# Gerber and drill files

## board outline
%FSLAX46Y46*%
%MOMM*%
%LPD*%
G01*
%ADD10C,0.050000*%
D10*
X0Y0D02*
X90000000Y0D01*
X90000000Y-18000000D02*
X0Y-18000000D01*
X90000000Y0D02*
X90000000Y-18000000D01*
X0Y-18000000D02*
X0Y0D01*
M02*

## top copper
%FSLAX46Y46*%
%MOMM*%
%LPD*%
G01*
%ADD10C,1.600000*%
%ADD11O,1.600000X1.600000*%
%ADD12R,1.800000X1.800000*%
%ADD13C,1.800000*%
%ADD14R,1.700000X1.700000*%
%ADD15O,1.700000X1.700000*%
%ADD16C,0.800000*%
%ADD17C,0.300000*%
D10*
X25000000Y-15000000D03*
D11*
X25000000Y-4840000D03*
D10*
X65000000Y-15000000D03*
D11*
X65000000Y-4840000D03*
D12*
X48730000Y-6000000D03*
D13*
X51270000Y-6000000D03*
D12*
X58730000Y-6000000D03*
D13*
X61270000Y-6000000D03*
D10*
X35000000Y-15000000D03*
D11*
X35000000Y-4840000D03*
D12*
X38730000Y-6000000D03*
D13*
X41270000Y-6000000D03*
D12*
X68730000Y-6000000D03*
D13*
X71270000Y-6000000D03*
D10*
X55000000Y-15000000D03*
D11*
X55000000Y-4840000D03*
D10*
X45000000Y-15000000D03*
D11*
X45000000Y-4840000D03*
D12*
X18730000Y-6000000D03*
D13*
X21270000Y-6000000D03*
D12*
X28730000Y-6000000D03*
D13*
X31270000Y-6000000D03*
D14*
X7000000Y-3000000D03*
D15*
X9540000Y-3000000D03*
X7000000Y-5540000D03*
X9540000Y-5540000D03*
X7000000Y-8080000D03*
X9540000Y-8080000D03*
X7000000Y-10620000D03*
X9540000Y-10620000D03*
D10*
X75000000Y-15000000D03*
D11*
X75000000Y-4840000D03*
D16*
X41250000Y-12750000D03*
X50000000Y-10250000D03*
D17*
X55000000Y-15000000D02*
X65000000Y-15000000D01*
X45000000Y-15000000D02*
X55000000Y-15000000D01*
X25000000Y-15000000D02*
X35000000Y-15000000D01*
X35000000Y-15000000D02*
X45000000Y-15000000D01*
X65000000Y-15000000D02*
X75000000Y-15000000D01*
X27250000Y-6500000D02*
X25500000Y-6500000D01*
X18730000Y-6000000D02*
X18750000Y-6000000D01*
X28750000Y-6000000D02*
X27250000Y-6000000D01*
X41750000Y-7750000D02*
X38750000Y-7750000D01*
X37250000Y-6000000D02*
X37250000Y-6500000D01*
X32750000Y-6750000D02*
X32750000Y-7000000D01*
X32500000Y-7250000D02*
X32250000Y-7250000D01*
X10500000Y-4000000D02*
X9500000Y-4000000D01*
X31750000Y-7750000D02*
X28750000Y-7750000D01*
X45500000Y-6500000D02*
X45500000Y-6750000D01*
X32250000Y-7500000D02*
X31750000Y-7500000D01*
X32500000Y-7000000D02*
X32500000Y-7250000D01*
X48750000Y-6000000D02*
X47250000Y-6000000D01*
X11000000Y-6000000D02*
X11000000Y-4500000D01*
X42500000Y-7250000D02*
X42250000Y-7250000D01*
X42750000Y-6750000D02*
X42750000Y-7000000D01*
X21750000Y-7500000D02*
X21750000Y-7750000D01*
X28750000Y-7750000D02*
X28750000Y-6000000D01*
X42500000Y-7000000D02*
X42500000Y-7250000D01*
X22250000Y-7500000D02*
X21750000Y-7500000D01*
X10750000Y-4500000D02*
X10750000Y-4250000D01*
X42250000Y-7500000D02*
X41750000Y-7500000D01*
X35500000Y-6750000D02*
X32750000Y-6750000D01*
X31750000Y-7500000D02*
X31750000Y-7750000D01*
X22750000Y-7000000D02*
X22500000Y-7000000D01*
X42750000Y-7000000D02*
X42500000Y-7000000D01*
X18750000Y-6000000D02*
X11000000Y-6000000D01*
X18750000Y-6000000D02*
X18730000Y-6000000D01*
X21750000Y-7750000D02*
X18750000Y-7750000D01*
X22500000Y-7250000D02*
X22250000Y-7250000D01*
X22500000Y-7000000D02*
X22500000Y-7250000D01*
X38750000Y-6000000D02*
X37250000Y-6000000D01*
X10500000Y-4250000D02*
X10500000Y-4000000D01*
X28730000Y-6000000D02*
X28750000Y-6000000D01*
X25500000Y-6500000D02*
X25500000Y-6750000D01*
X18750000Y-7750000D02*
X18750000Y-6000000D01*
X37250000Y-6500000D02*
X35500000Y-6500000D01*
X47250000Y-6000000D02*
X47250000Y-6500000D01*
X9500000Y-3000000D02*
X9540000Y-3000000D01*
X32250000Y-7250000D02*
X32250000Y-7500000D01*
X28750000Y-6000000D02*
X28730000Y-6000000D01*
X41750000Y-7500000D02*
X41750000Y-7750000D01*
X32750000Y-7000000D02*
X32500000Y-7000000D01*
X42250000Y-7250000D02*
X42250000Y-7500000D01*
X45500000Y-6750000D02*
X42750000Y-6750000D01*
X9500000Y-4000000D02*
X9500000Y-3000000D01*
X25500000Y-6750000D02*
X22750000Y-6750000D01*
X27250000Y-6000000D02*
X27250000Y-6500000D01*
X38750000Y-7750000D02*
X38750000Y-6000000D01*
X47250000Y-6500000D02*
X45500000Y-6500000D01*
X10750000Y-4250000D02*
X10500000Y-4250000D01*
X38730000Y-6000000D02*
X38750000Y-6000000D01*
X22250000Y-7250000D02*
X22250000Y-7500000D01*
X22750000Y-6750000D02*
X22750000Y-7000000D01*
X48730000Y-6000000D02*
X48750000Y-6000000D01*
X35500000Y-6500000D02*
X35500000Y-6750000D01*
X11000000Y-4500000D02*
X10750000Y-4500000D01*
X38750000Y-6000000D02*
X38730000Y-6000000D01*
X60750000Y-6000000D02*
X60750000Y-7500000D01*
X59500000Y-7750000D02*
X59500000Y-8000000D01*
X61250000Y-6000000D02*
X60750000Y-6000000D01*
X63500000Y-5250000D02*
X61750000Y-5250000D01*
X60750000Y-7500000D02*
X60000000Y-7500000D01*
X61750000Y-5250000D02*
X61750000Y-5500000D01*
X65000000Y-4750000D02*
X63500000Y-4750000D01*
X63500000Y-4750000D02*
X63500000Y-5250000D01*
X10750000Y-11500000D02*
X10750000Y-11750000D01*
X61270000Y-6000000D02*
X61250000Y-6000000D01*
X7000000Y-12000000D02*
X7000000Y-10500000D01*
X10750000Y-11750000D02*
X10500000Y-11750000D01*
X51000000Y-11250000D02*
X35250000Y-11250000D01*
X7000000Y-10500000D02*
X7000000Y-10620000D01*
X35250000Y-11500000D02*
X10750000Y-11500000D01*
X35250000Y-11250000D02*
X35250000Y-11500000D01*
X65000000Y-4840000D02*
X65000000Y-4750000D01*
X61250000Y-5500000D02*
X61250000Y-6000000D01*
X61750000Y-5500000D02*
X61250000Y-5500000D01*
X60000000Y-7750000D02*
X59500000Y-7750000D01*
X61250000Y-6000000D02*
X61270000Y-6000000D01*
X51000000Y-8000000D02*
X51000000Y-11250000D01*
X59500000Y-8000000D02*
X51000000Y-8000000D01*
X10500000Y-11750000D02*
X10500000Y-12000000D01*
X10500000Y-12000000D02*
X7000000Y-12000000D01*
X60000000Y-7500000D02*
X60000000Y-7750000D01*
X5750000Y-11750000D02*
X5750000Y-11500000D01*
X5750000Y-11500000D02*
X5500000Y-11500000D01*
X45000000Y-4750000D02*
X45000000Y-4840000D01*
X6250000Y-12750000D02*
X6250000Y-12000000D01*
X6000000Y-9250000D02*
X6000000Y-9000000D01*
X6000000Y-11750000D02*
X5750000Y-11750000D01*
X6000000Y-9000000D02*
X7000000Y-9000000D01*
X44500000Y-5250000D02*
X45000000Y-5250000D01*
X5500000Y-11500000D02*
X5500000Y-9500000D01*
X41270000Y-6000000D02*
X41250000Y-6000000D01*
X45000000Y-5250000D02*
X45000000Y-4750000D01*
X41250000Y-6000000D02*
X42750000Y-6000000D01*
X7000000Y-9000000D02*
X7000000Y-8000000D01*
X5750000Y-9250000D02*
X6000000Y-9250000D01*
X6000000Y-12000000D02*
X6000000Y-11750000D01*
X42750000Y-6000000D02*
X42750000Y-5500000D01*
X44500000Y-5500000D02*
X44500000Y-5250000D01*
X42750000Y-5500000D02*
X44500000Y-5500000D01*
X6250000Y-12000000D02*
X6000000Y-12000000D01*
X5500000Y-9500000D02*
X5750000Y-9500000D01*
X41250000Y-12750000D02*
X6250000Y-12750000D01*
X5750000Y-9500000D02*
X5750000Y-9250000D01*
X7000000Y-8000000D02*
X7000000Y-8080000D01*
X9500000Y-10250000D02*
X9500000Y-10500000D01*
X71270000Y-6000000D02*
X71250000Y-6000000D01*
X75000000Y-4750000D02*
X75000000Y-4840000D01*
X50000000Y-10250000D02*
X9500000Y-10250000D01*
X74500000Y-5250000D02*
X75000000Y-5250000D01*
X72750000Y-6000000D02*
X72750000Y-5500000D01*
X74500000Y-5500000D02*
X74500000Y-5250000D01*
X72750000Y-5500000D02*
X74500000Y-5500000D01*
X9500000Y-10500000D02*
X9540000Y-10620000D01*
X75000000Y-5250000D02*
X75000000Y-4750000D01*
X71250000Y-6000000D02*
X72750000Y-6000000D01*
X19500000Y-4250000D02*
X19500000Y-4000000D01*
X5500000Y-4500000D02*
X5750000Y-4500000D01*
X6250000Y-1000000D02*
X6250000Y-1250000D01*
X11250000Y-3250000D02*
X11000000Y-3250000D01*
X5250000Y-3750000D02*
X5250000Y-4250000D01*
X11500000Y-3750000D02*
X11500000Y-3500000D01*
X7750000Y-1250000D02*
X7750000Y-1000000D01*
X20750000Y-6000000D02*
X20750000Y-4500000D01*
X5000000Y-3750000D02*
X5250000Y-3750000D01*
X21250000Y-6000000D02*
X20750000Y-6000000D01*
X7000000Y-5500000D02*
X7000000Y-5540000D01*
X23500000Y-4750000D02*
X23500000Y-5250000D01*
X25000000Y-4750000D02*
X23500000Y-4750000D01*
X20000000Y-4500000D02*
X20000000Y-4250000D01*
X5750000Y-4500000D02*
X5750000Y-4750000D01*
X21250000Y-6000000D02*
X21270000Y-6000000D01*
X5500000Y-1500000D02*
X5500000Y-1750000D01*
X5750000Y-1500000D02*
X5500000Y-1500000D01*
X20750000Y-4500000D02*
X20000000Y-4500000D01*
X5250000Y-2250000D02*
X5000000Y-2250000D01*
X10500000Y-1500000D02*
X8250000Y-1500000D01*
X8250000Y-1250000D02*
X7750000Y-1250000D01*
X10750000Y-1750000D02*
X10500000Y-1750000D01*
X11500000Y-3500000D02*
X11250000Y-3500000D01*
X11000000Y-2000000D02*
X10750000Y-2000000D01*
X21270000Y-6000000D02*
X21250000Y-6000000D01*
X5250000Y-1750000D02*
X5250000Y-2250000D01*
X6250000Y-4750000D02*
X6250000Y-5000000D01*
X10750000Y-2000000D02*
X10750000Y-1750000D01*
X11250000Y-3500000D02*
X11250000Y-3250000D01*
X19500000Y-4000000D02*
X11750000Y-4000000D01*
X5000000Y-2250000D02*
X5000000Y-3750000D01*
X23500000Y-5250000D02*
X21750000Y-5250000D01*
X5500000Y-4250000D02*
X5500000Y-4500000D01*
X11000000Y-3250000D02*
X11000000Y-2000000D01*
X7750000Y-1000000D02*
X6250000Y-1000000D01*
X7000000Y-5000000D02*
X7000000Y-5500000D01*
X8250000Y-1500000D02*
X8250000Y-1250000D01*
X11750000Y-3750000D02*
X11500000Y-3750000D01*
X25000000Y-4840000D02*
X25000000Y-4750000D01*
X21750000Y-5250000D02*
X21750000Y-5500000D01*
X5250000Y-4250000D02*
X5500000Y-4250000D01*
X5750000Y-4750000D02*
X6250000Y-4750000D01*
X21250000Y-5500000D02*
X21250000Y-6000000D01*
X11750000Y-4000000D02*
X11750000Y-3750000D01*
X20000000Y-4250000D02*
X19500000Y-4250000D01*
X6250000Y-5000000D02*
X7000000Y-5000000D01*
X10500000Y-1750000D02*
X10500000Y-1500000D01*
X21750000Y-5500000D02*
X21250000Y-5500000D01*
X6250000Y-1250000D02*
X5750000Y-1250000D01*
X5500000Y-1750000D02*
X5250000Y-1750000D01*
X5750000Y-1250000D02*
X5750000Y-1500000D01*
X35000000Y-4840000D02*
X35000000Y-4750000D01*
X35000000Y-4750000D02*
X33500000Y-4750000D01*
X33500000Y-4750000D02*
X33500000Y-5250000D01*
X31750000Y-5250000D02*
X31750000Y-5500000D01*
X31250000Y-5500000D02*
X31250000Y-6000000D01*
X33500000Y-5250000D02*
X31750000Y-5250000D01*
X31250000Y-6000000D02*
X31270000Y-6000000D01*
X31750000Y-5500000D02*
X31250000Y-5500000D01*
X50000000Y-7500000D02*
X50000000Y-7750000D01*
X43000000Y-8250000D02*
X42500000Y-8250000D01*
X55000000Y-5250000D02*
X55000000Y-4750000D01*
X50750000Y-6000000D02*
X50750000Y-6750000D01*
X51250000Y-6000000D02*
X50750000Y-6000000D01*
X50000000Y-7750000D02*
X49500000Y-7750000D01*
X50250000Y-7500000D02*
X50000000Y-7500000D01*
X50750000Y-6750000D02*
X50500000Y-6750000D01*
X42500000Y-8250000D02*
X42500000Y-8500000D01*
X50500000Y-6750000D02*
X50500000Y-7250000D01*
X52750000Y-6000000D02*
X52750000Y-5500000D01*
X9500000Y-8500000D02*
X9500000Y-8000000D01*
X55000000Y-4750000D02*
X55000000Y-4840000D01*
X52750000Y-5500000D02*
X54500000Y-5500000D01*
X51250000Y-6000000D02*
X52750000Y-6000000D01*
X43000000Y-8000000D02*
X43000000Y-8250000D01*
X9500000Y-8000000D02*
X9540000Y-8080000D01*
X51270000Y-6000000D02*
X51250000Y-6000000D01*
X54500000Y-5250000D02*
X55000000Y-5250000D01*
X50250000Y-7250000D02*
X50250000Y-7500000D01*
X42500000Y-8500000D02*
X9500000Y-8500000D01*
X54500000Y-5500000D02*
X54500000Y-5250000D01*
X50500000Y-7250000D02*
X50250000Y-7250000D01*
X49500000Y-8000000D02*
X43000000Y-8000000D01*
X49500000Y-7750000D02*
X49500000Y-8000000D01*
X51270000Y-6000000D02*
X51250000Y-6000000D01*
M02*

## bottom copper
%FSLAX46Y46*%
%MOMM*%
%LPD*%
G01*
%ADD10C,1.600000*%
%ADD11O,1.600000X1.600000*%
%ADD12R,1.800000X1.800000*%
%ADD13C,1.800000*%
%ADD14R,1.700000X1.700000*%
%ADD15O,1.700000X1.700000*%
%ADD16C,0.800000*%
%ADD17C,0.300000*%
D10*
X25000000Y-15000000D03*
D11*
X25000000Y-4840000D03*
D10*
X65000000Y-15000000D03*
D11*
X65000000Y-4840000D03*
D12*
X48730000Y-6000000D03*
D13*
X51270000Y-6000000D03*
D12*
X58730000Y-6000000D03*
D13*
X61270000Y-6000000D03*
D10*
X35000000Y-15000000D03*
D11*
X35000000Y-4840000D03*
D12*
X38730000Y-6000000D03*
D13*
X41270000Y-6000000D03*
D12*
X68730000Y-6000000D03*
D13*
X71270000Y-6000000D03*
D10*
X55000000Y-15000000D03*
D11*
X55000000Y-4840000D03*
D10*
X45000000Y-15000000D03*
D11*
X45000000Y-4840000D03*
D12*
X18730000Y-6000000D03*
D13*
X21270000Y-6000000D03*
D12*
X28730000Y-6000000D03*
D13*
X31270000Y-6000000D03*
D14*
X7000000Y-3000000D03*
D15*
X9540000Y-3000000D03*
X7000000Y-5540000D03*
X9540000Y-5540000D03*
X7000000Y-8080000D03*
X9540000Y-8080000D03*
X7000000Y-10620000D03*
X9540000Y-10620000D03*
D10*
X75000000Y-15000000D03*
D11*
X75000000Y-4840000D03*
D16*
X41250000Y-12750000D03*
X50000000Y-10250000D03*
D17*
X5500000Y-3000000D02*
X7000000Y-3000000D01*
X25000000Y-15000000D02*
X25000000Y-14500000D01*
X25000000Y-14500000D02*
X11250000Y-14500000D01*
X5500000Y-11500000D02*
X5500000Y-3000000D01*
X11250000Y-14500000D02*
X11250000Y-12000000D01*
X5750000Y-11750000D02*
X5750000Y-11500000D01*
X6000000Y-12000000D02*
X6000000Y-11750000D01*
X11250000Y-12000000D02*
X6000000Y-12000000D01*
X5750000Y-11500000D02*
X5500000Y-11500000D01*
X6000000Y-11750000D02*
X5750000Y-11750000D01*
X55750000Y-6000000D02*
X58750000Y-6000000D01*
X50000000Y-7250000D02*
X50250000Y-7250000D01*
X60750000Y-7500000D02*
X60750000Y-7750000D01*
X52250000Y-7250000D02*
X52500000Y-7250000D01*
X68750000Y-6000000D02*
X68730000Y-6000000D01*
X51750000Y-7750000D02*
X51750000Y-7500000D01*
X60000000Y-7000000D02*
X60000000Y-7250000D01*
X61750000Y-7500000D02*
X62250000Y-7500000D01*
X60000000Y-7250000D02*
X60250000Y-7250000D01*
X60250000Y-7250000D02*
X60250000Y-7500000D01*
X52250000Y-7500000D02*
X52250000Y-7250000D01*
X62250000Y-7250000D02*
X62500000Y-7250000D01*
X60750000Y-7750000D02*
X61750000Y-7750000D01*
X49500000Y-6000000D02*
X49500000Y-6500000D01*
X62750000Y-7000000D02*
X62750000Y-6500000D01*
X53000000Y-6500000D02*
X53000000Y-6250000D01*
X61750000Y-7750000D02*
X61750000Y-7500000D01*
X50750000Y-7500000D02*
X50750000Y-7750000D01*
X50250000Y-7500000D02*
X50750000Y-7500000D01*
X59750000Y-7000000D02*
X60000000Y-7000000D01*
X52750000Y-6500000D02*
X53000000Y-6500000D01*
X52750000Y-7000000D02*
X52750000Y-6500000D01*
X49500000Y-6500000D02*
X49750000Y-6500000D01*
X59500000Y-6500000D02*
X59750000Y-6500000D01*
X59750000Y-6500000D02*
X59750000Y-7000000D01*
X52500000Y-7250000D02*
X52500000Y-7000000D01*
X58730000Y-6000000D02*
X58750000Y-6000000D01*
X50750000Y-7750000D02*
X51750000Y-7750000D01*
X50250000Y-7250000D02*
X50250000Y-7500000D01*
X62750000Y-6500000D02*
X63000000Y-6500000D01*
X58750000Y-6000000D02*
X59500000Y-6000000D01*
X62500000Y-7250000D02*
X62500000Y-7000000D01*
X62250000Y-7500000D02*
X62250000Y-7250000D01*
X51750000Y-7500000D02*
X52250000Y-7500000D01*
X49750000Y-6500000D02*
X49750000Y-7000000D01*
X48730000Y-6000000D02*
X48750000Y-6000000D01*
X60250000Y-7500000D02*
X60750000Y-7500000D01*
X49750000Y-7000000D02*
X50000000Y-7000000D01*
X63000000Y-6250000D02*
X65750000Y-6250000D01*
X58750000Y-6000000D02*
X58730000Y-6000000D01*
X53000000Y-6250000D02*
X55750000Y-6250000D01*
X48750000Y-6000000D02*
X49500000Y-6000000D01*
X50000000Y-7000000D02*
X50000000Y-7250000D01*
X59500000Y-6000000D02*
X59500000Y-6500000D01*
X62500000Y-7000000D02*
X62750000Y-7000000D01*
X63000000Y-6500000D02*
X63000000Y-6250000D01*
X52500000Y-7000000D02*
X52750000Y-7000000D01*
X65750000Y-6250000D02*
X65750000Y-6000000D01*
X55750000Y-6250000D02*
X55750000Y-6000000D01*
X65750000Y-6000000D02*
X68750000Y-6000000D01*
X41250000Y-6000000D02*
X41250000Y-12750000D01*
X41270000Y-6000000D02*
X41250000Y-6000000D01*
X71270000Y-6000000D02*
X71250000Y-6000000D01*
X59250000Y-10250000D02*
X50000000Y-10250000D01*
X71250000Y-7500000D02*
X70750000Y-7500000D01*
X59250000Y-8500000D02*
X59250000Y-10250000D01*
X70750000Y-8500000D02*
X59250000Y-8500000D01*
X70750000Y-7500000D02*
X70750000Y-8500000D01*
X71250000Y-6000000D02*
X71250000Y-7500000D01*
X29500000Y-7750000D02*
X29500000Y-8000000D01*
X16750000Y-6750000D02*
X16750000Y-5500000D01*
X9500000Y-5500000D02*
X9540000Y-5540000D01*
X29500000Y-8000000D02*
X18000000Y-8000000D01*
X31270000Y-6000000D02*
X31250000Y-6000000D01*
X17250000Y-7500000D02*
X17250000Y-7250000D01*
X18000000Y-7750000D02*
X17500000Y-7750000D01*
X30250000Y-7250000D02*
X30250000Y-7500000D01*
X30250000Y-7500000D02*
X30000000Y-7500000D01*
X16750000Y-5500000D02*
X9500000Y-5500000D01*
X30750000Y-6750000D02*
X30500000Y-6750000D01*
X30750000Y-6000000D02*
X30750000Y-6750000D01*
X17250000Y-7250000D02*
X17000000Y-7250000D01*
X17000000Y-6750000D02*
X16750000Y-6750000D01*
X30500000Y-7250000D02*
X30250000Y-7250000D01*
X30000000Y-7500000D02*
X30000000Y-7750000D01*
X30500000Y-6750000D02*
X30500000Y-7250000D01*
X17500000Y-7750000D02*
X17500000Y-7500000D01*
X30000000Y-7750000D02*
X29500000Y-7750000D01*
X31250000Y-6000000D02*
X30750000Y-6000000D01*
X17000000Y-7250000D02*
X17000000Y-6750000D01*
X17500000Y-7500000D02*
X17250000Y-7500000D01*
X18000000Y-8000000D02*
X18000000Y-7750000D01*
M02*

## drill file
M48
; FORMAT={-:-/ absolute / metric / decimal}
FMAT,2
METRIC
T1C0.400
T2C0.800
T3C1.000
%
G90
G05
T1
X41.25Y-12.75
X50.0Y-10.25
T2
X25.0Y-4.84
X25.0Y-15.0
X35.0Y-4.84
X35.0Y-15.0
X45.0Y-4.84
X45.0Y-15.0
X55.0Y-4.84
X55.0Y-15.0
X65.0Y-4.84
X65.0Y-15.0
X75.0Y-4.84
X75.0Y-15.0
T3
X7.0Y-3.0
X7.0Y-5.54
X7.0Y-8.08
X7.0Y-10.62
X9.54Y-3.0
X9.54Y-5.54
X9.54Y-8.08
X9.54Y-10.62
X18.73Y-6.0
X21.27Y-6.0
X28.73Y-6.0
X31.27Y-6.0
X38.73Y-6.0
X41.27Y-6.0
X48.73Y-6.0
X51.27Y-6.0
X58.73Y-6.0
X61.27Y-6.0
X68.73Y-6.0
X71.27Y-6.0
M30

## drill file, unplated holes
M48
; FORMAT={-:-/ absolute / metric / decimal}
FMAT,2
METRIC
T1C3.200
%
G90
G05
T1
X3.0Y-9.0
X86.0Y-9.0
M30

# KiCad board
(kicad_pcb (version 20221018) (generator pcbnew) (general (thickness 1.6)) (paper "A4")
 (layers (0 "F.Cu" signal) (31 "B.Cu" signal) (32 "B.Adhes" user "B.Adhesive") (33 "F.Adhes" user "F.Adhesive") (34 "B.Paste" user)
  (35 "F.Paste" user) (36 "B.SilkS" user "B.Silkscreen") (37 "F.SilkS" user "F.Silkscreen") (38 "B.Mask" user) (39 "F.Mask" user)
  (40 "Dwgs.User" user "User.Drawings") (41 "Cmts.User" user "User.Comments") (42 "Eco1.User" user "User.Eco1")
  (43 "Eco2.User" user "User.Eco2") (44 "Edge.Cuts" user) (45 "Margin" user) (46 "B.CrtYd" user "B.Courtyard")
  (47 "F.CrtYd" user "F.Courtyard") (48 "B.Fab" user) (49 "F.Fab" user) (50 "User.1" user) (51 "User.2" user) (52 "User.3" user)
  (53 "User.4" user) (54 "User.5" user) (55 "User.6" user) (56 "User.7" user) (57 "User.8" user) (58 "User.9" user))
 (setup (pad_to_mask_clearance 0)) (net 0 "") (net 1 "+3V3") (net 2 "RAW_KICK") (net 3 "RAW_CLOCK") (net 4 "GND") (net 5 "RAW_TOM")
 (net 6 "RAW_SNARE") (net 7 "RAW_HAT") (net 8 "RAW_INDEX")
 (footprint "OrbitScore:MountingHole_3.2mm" (layer "F.Cu") (at 3 9)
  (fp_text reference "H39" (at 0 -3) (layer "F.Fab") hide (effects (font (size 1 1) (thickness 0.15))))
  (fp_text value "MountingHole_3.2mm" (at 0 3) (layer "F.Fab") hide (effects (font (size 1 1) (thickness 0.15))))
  (pad "" np_thru_hole circle (at 0 0) (size 3.2 3.2) (drill 3.2) (layers "*.Cu" "*.Mask")))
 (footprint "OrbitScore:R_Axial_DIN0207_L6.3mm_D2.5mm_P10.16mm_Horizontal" (layer "F.Cu") (at 25 15 90)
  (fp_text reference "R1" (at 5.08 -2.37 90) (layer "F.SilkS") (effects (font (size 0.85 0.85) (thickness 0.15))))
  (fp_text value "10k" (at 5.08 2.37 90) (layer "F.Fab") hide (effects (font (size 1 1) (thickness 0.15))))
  (pad "1" thru_hole circle (at 0 0 90) (size 1.6 1.6) (drill 0.8) (layers "*.Cu" "*.Mask") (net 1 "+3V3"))
  (pad "2" thru_hole oval (at 10.16 0 90) (size 1.6 1.6) (drill 0.8) (layers "*.Cu" "*.Mask") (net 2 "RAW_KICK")))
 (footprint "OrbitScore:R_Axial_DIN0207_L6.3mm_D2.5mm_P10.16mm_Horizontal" (layer "F.Cu") (at 65 15 90)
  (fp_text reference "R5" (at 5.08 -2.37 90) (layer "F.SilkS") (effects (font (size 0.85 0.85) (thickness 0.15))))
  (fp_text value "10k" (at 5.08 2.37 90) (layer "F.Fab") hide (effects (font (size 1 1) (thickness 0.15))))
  (pad "1" thru_hole circle (at 0 0 90) (size 1.6 1.6) (drill 0.8) (layers "*.Cu" "*.Mask") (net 1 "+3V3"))
  (pad "2" thru_hole oval (at 10.16 0 90) (size 1.6 1.6) (drill 0.8) (layers "*.Cu" "*.Mask") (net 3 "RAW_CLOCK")))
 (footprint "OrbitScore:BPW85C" (layer "F.Cu") (at 50 6)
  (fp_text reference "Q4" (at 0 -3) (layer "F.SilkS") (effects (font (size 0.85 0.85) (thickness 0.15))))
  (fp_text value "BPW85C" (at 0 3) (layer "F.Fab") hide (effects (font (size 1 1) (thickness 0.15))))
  (pad "1" thru_hole rect (at -1.27 0) (size 1.8 1.8) (drill 1) (layers "*.Cu" "*.Mask") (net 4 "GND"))
  (pad "2" thru_hole circle (at 1.27 0) (size 1.8 1.8) (drill 1) (layers "*.Cu" "*.Mask") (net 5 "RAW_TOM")))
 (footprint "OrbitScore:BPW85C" (layer "F.Cu") (at 60 6)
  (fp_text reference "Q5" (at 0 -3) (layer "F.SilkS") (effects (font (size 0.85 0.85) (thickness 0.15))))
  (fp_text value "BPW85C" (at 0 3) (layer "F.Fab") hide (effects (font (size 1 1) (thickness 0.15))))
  (pad "1" thru_hole rect (at -1.27 0) (size 1.8 1.8) (drill 1) (layers "*.Cu" "*.Mask") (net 4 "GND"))
  (pad "2" thru_hole circle (at 1.27 0) (size 1.8 1.8) (drill 1) (layers "*.Cu" "*.Mask") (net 3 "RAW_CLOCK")))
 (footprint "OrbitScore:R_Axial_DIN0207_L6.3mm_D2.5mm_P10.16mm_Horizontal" (layer "F.Cu") (at 35 15 90)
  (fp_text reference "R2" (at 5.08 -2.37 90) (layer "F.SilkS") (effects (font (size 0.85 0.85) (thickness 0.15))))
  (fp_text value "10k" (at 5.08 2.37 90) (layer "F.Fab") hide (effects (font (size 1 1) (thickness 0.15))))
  (pad "1" thru_hole circle (at 0 0 90) (size 1.6 1.6) (drill 0.8) (layers "*.Cu" "*.Mask") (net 1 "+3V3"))
  (pad "2" thru_hole oval (at 10.16 0 90) (size 1.6 1.6) (drill 0.8) (layers "*.Cu" "*.Mask") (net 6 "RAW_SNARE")))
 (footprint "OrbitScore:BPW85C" (layer "F.Cu") (at 40 6)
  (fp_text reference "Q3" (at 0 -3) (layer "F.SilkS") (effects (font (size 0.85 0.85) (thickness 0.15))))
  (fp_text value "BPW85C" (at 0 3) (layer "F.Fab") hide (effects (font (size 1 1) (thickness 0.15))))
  (pad "1" thru_hole rect (at -1.27 0) (size 1.8 1.8) (drill 1) (layers "*.Cu" "*.Mask") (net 4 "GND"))
  (pad "2" thru_hole circle (at 1.27 0) (size 1.8 1.8) (drill 1) (layers "*.Cu" "*.Mask") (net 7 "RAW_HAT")))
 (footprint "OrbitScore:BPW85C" (layer "F.Cu") (at 70 6)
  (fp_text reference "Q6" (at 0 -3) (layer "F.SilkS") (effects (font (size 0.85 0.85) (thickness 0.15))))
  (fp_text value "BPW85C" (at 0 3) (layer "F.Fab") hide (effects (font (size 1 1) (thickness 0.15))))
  (pad "1" thru_hole rect (at -1.27 0) (size 1.8 1.8) (drill 1) (layers "*.Cu" "*.Mask") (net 4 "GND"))
  (pad "2" thru_hole circle (at 1.27 0) (size 1.8 1.8) (drill 1) (layers "*.Cu" "*.Mask") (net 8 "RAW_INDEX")))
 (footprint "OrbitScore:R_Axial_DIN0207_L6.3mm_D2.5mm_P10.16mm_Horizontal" (layer "F.Cu") (at 55 15 90)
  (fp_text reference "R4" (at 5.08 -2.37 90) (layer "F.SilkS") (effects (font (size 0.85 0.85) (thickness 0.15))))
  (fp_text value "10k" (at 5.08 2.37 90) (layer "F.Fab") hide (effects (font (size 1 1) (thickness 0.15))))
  (pad "1" thru_hole circle (at 0 0 90) (size 1.6 1.6) (drill 0.8) (layers "*.Cu" "*.Mask") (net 1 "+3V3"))
  (pad "2" thru_hole oval (at 10.16 0 90) (size 1.6 1.6) (drill 0.8) (layers "*.Cu" "*.Mask") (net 5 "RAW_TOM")))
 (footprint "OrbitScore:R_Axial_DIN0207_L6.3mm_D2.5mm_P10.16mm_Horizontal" (layer "F.Cu") (at 45 15 90)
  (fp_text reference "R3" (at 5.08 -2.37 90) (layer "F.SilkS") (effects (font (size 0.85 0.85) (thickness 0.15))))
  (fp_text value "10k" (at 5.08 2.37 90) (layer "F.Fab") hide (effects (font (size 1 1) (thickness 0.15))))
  (pad "1" thru_hole circle (at 0 0 90) (size 1.6 1.6) (drill 0.8) (layers "*.Cu" "*.Mask") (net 1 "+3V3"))
  (pad "2" thru_hole oval (at 10.16 0 90) (size 1.6 1.6) (drill 0.8) (layers "*.Cu" "*.Mask") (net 7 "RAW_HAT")))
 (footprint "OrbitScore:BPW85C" (layer "F.Cu") (at 20 6)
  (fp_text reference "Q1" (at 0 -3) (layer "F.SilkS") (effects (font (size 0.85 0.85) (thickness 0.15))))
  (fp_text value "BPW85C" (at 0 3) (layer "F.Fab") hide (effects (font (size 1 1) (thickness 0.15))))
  (pad "1" thru_hole rect (at -1.27 0) (size 1.8 1.8) (drill 1) (layers "*.Cu" "*.Mask") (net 4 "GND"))
  (pad "2" thru_hole circle (at 1.27 0) (size 1.8 1.8) (drill 1) (layers "*.Cu" "*.Mask") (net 2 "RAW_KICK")))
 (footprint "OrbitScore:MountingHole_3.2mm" (layer "F.Cu") (at 86 9)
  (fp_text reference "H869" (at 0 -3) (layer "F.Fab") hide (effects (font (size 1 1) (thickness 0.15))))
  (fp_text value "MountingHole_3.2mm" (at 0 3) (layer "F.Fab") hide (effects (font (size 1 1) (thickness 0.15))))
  (pad "" np_thru_hole circle (at 0 0) (size 3.2 3.2) (drill 3.2) (layers "*.Cu" "*.Mask")))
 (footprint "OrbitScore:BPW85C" (layer "F.Cu") (at 30 6)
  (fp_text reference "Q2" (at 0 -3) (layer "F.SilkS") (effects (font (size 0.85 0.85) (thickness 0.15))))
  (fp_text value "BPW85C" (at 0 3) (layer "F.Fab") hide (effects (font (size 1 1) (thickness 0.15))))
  (pad "1" thru_hole rect (at -1.27 0) (size 1.8 1.8) (drill 1) (layers "*.Cu" "*.Mask") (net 4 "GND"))
  (pad "2" thru_hole circle (at 1.27 0) (size 1.8 1.8) (drill 1) (layers "*.Cu" "*.Mask") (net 6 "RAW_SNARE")))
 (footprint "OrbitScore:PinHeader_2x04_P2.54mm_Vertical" (layer "F.Cu") (at 7 3)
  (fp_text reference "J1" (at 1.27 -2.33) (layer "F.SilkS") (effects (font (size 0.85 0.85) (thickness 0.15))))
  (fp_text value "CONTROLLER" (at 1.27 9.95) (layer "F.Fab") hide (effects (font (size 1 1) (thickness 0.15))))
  (pad "1" thru_hole rect (at 0 0) (size 1.7 1.7) (drill 1) (layers "*.Cu" "*.Mask") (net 1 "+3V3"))
  (pad "2" thru_hole oval (at 2.54 0) (size 1.7 1.7) (drill 1) (layers "*.Cu" "*.Mask") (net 4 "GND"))
  (pad "3" thru_hole oval (at 0 2.54) (size 1.7 1.7) (drill 1) (layers "*.Cu" "*.Mask") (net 2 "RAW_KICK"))
  (pad "4" thru_hole oval (at 2.54 2.54) (size 1.7 1.7) (drill 1) (layers "*.Cu" "*.Mask") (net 6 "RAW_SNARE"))
  (pad "5" thru_hole oval (at 0 5.08) (size 1.7 1.7) (drill 1) (layers "*.Cu" "*.Mask") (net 7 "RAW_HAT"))
  (pad "6" thru_hole oval (at 2.54 5.08) (size 1.7 1.7) (drill 1) (layers "*.Cu" "*.Mask") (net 5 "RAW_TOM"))
  (pad "7" thru_hole oval (at 0 7.62) (size 1.7 1.7) (drill 1) (layers "*.Cu" "*.Mask") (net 3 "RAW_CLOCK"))
  (pad "8" thru_hole oval (at 2.54 7.62) (size 1.7 1.7) (drill 1) (layers "*.Cu" "*.Mask") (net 8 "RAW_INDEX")))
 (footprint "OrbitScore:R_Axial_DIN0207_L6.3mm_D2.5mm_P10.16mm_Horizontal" (layer "F.Cu") (at 75 15 90)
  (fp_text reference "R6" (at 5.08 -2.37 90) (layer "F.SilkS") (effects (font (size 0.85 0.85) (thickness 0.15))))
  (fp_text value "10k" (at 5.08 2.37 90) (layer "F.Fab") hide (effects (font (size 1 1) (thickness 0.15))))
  (pad "1" thru_hole circle (at 0 0 90) (size 1.6 1.6) (drill 0.8) (layers "*.Cu" "*.Mask") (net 1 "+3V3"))
  (pad "2" thru_hole oval (at 10.16 0 90) (size 1.6 1.6) (drill 0.8) (layers "*.Cu" "*.Mask") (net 8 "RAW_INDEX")))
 (gr_line (start 0 0) (end 90 0) (stroke (width 0.05) (type default)) (layer "Edge.Cuts"))
 (gr_line (start 90 18) (end 0 18) (stroke (width 0.05) (type default)) (layer "Edge.Cuts"))
 (gr_line (start 90 0) (end 90 18) (stroke (width 0.05) (type default)) (layer "Edge.Cuts"))
 (gr_line (start 0 18) (end 0 0) (stroke (width 0.05) (type default)) (layer "Edge.Cuts"))
 (segment (start 55 15) (end 65 15) (width 0.3) (layer "F.Cu") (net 1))
 (segment (start 45 15) (end 55 15) (width 0.3) (layer "F.Cu") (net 1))
 (segment (start 25 15) (end 35 15) (width 0.3) (layer "F.Cu") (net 1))
 (segment (start 35 15) (end 45 15) (width 0.3) (layer "F.Cu") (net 1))
 (segment (start 65 15) (end 75 15) (width 0.3) (layer "F.Cu") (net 1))
 (segment (start 5.5 3) (end 7 3) (width 0.3) (layer "B.Cu") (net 1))
 (segment (start 25 15) (end 25 14.5) (width 0.3) (layer "B.Cu") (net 1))
 (segment (start 25 14.5) (end 11.25 14.5) (width 0.3) (layer "B.Cu") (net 1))
 (segment (start 5.5 11.5) (end 5.5 3) (width 0.3) (layer "B.Cu") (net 1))
 (segment (start 11.25 14.5) (end 11.25 12) (width 0.3) (layer "B.Cu") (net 1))
 (segment (start 5.75 11.75) (end 5.75 11.5) (width 0.3) (layer "B.Cu") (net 1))
 (segment (start 6 12) (end 6 11.75) (width 0.3) (layer "B.Cu") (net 1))
 (segment (start 11.25 12) (end 6 12) (width 0.3) (layer "B.Cu") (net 1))
 (segment (start 5.75 11.5) (end 5.5 11.5) (width 0.3) (layer "B.Cu") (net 1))
 (segment (start 6 11.75) (end 5.75 11.75) (width 0.3) (layer "B.Cu") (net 1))
 (segment (start 27.25 6.5) (end 25.5 6.5) (width 0.3) (layer "F.Cu") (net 4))
 (segment (start 18.73 6) (end 18.75 6) (width 0.3) (layer "F.Cu") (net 4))
 (segment (start 28.75 6) (end 27.25 6) (width 0.3) (layer "F.Cu") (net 4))
 (segment (start 41.75 7.75) (end 38.75 7.75) (width 0.3) (layer "F.Cu") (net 4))
 (segment (start 37.25 6) (end 37.25 6.5) (width 0.3) (layer "F.Cu") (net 4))
 (segment (start 32.75 6.75) (end 32.75 7) (width 0.3) (layer "F.Cu") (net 4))
 (segment (start 32.5 7.25) (end 32.25 7.25) (width 0.3) (layer "F.Cu") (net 4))
 (segment (start 10.5 4) (end 9.5 4) (width 0.3) (layer "F.Cu") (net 4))
 (segment (start 31.75 7.75) (end 28.75 7.75) (width 0.3) (layer "F.Cu") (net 4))
 (segment (start 45.5 6.5) (end 45.5 6.75) (width 0.3) (layer "F.Cu") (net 4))
 (segment (start 32.25 7.5) (end 31.75 7.5) (width 0.3) (layer "F.Cu") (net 4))
 (segment (start 32.5 7) (end 32.5 7.25) (width 0.3) (layer "F.Cu") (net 4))
 (segment (start 48.75 6) (end 47.25 6) (width 0.3) (layer "F.Cu") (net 4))
 (segment (start 11 6) (end 11 4.5) (width 0.3) (layer "F.Cu") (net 4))
 (segment (start 42.5 7.25) (end 42.25 7.25) (width 0.3) (layer "F.Cu") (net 4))
 (segment (start 42.75 6.75) (end 42.75 7) (width 0.3) (layer "F.Cu") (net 4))
 (segment (start 21.75 7.5) (end 21.75 7.75) (width 0.3) (layer "F.Cu") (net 4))
 (segment (start 28.75 7.75) (end 28.75 6) (width 0.3) (layer "F.Cu") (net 4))
 (segment (start 42.5 7) (end 42.5 7.25) (width 0.3) (layer "F.Cu") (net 4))
 (segment (start 22.25 7.5) (end 21.75 7.5) (width 0.3) (layer "F.Cu") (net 4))
 (segment (start 10.75 4.5) (end 10.75 4.25) (width 0.3) (layer "F.Cu") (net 4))
 (segment (start 42.25 7.5) (end 41.75 7.5) (width 0.3) (layer "F.Cu") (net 4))
 (segment (start 35.5 6.75) (end 32.75 6.75) (width 0.3) (layer "F.Cu") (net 4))
 (segment (start 31.75 7.5) (end 31.75 7.75) (width 0.3) (layer "F.Cu") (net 4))
 (segment (start 22.75 7) (end 22.5 7) (width 0.3) (layer "F.Cu") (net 4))
 (segment (start 42.75 7) (end 42.5 7) (width 0.3) (layer "F.Cu") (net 4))
 (segment (start 18.75 6) (end 11 6) (width 0.3) (layer "F.Cu") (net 4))
 (segment (start 18.75 6) (end 18.73 6) (width 0.3) (layer "F.Cu") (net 4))
 (segment (start 21.75 7.75) (end 18.75 7.75) (width 0.3) (layer "F.Cu") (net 4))
 (segment (start 22.5 7.25) (end 22.25 7.25) (width 0.3) (layer "F.Cu") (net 4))
 (segment (start 22.5 7) (end 22.5 7.25) (width 0.3) (layer "F.Cu") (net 4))
 (segment (start 38.75 6) (end 37.25 6) (width 0.3) (layer "F.Cu") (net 4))
 (segment (start 10.5 4.25) (end 10.5 4) (width 0.3) (layer "F.Cu") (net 4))
 (segment (start 28.73 6) (end 28.75 6) (width 0.3) (layer "F.Cu") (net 4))
 (segment (start 25.5 6.5) (end 25.5 6.75) (width 0.3) (layer "F.Cu") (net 4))
 (segment (start 18.75 7.75) (end 18.75 6) (width 0.3) (layer "F.Cu") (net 4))
 (segment (start 37.25 6.5) (end 35.5 6.5) (width 0.3) (layer "F.Cu") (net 4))
 (segment (start 47.25 6) (end 47.25 6.5) (width 0.3) (layer "F.Cu") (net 4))
 (segment (start 9.5 3) (end 9.54 3) (width 0.3) (layer "F.Cu") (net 4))
 (segment (start 32.25 7.25) (end 32.25 7.5) (width 0.3) (layer "F.Cu") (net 4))
 (segment (start 28.75 6) (end 28.73 6) (width 0.3) (layer "F.Cu") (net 4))
 (segment (start 41.75 7.5) (end 41.75 7.75) (width 0.3) (layer "F.Cu") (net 4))
 (segment (start 32.75 7) (end 32.5 7) (width 0.3) (layer "F.Cu") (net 4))
 (segment (start 42.25 7.25) (end 42.25 7.5) (width 0.3) (layer "F.Cu") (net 4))
 (segment (start 45.5 6.75) (end 42.75 6.75) (width 0.3) (layer "F.Cu") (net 4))
 (segment (start 9.5 4) (end 9.5 3) (width 0.3) (layer "F.Cu") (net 4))
 (segment (start 25.5 6.75) (end 22.75 6.75) (width 0.3) (layer "F.Cu") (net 4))
 (segment (start 27.25 6) (end 27.25 6.5) (width 0.3) (layer "F.Cu") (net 4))
 (segment (start 38.75 7.75) (end 38.75 6) (width 0.3) (layer "F.Cu") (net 4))
 (segment (start 47.25 6.5) (end 45.5 6.5) (width 0.3) (layer "F.Cu") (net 4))
 (segment (start 10.75 4.25) (end 10.5 4.25) (width 0.3) (layer "F.Cu") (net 4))
 (segment (start 38.73 6) (end 38.75 6) (width 0.3) (layer "F.Cu") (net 4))
 (segment (start 22.25 7.25) (end 22.25 7.5) (width 0.3) (layer "F.Cu") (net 4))
 (segment (start 22.75 6.75) (end 22.75 7) (width 0.3) (layer "F.Cu") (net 4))
 (segment (start 48.73 6) (end 48.75 6) (width 0.3) (layer "F.Cu") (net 4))
 (segment (start 35.5 6.5) (end 35.5 6.75) (width 0.3) (layer "F.Cu") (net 4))
 (segment (start 11 4.5) (end 10.75 4.5) (width 0.3) (layer "F.Cu") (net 4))
 (segment (start 38.75 6) (end 38.73 6) (width 0.3) (layer "F.Cu") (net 4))
 (segment (start 55.75 6) (end 58.75 6) (width 0.3) (layer "B.Cu") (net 4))
 (segment (start 50 7.25) (end 50.25 7.25) (width 0.3) (layer "B.Cu") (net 4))
 (segment (start 60.75 7.5) (end 60.75 7.75) (width 0.3) (layer "B.Cu") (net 4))
 (segment (start 52.25 7.25) (end 52.5 7.25) (width 0.3) (layer "B.Cu") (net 4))
 (segment (start 68.75 6) (end 68.73 6) (width 0.3) (layer "B.Cu") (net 4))
 (segment (start 51.75 7.75) (end 51.75 7.5) (width 0.3) (layer "B.Cu") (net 4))
 (segment (start 60 7) (end 60 7.25) (width 0.3) (layer "B.Cu") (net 4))
 (segment (start 61.75 7.5) (end 62.25 7.5) (width 0.3) (layer "B.Cu") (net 4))
 (segment (start 60 7.25) (end 60.25 7.25) (width 0.3) (layer "B.Cu") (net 4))
 (segment (start 60.25 7.25) (end 60.25 7.5) (width 0.3) (layer "B.Cu") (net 4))
 (segment (start 52.25 7.5) (end 52.25 7.25) (width 0.3) (layer "B.Cu") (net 4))
 (segment (start 62.25 7.25) (end 62.5 7.25) (width 0.3) (layer "B.Cu") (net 4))
 (segment (start 60.75 7.75) (end 61.75 7.75) (width 0.3) (layer "B.Cu") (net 4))
 (segment (start 49.5 6) (end 49.5 6.5) (width 0.3) (layer "B.Cu") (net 4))
 (segment (start 62.75 7) (end 62.75 6.5) (width 0.3) (layer "B.Cu") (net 4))
 (segment (start 53 6.5) (end 53 6.25) (width 0.3) (layer "B.Cu") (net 4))
 (segment (start 61.75 7.75) (end 61.75 7.5) (width 0.3) (layer "B.Cu") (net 4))
 (segment (start 50.75 7.5) (end 50.75 7.75) (width 0.3) (layer "B.Cu") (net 4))
 (segment (start 50.25 7.5) (end 50.75 7.5) (width 0.3) (layer "B.Cu") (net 4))
 (segment (start 59.75 7) (end 60 7) (width 0.3) (layer "B.Cu") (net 4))
 (segment (start 52.75 6.5) (end 53 6.5) (width 0.3) (layer "B.Cu") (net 4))
 (segment (start 52.75 7) (end 52.75 6.5) (width 0.3) (layer "B.Cu") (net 4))
 (segment (start 49.5 6.5) (end 49.75 6.5) (width 0.3) (layer "B.Cu") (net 4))
 (segment (start 59.5 6.5) (end 59.75 6.5) (width 0.3) (layer "B.Cu") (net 4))
 (segment (start 59.75 6.5) (end 59.75 7) (width 0.3) (layer "B.Cu") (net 4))
 (segment (start 52.5 7.25) (end 52.5 7) (width 0.3) (layer "B.Cu") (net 4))
 (segment (start 58.73 6) (end 58.75 6) (width 0.3) (layer "B.Cu") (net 4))
 (segment (start 50.75 7.75) (end 51.75 7.75) (width 0.3) (layer "B.Cu") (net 4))
 (segment (start 50.25 7.25) (end 50.25 7.5) (width 0.3) (layer "B.Cu") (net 4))
 (segment (start 62.75 6.5) (end 63 6.5) (width 0.3) (layer "B.Cu") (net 4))
 (segment (start 58.75 6) (end 59.5 6) (width 0.3) (layer "B.Cu") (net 4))
 (segment (start 62.5 7.25) (end 62.5 7) (width 0.3) (layer "B.Cu") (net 4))
 (segment (start 62.25 7.5) (end 62.25 7.25) (width 0.3) (layer "B.Cu") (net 4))
 (segment (start 51.75 7.5) (end 52.25 7.5) (width 0.3) (layer "B.Cu") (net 4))
 (segment (start 49.75 6.5) (end 49.75 7) (width 0.3) (layer "B.Cu") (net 4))
 (segment (start 48.73 6) (end 48.75 6) (width 0.3) (layer "B.Cu") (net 4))
 (segment (start 60.25 7.5) (end 60.75 7.5) (width 0.3) (layer "B.Cu") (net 4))
 (segment (start 49.75 7) (end 50 7) (width 0.3) (layer "B.Cu") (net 4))
 (segment (start 63 6.25) (end 65.75 6.25) (width 0.3) (layer "B.Cu") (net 4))
 (segment (start 58.75 6) (end 58.73 6) (width 0.3) (layer "B.Cu") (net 4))
 (segment (start 53 6.25) (end 55.75 6.25) (width 0.3) (layer "B.Cu") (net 4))
 (segment (start 48.75 6) (end 49.5 6) (width 0.3) (layer "B.Cu") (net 4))
 (segment (start 50 7) (end 50 7.25) (width 0.3) (layer "B.Cu") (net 4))
 (segment (start 59.5 6) (end 59.5 6.5) (width 0.3) (layer "B.Cu") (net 4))
 (segment (start 62.5 7) (end 62.75 7) (width 0.3) (layer "B.Cu") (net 4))
 (segment (start 63 6.5) (end 63 6.25) (width 0.3) (layer "B.Cu") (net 4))
 (segment (start 52.5 7) (end 52.75 7) (width 0.3) (layer "B.Cu") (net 4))
 (segment (start 65.75 6.25) (end 65.75 6) (width 0.3) (layer "B.Cu") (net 4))
 (segment (start 55.75 6.25) (end 55.75 6) (width 0.3) (layer "B.Cu") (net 4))
 (segment (start 65.75 6) (end 68.75 6) (width 0.3) (layer "B.Cu") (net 4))
 (segment (start 60.75 6) (end 60.75 7.5) (width 0.3) (layer "F.Cu") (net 3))
 (segment (start 59.5 7.75) (end 59.5 8) (width 0.3) (layer "F.Cu") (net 3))
 (segment (start 61.25 6) (end 60.75 6) (width 0.3) (layer "F.Cu") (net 3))
 (segment (start 63.5 5.25) (end 61.75 5.25) (width 0.3) (layer "F.Cu") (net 3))
 (segment (start 60.75 7.5) (end 60 7.5) (width 0.3) (layer "F.Cu") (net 3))
 (segment (start 61.75 5.25) (end 61.75 5.5) (width 0.3) (layer "F.Cu") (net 3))
 (segment (start 65 4.75) (end 63.5 4.75) (width 0.3) (layer "F.Cu") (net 3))
 (segment (start 63.5 4.75) (end 63.5 5.25) (width 0.3) (layer "F.Cu") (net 3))
 (segment (start 10.75 11.5) (end 10.75 11.75) (width 0.3) (layer "F.Cu") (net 3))
 (segment (start 61.27 6) (end 61.25 6) (width 0.3) (layer "F.Cu") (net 3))
 (segment (start 7 12) (end 7 10.5) (width 0.3) (layer "F.Cu") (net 3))
 (segment (start 10.75 11.75) (end 10.5 11.75) (width 0.3) (layer "F.Cu") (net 3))
 (segment (start 51 11.25) (end 35.25 11.25) (width 0.3) (layer "F.Cu") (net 3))
 (segment (start 7 10.5) (end 7 10.62) (width 0.3) (layer "F.Cu") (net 3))
 (segment (start 35.25 11.5) (end 10.75 11.5) (width 0.3) (layer "F.Cu") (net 3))
 (segment (start 35.25 11.25) (end 35.25 11.5) (width 0.3) (layer "F.Cu") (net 3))
 (segment (start 65 4.84) (end 65 4.75) (width 0.3) (layer "F.Cu") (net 3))
 (segment (start 61.25 5.5) (end 61.25 6) (width 0.3) (layer "F.Cu") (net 3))
 (segment (start 61.75 5.5) (end 61.25 5.5) (width 0.3) (layer "F.Cu") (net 3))
 (segment (start 60 7.75) (end 59.5 7.75) (width 0.3) (layer "F.Cu") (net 3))
 (segment (start 61.25 6) (end 61.27 6) (width 0.3) (layer "F.Cu") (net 3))
 (segment (start 51 8) (end 51 11.25) (width 0.3) (layer "F.Cu") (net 3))
 (segment (start 59.5 8) (end 51 8) (width 0.3) (layer "F.Cu") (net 3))
 (segment (start 10.5 11.75) (end 10.5 12) (width 0.3) (layer "F.Cu") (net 3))
 (segment (start 10.5 12) (end 7 12) (width 0.3) (layer "F.Cu") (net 3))
 (segment (start 60 7.5) (end 60 7.75) (width 0.3) (layer "F.Cu") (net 3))
 (segment (start 5.75 11.75) (end 5.75 11.5) (width 0.3) (layer "F.Cu") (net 7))
 (segment (start 5.75 11.5) (end 5.5 11.5) (width 0.3) (layer "F.Cu") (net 7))
 (segment (start 45 4.75) (end 45 4.84) (width 0.3) (layer "F.Cu") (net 7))
 (segment (start 6.25 12.75) (end 6.25 12) (width 0.3) (layer "F.Cu") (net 7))
 (segment (start 6 9.25) (end 6 9) (width 0.3) (layer "F.Cu") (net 7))
 (segment (start 6 11.75) (end 5.75 11.75) (width 0.3) (layer "F.Cu") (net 7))
 (segment (start 6 9) (end 7 9) (width 0.3) (layer "F.Cu") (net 7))
 (segment (start 44.5 5.25) (end 45 5.25) (width 0.3) (layer "F.Cu") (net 7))
 (segment (start 5.5 11.5) (end 5.5 9.5) (width 0.3) (layer "F.Cu") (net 7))
 (segment (start 41.27 6) (end 41.25 6) (width 0.3) (layer "F.Cu") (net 7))
 (segment (start 45 5.25) (end 45 4.75) (width 0.3) (layer "F.Cu") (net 7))
 (segment (start 41.25 6) (end 42.75 6) (width 0.3) (layer "F.Cu") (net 7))
 (segment (start 7 9) (end 7 8) (width 0.3) (layer "F.Cu") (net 7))
 (segment (start 5.75 9.25) (end 6 9.25) (width 0.3) (layer "F.Cu") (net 7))
 (segment (start 6 12) (end 6 11.75) (width 0.3) (layer "F.Cu") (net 7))
 (segment (start 42.75 6) (end 42.75 5.5) (width 0.3) (layer "F.Cu") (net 7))
 (segment (start 44.5 5.5) (end 44.5 5.25) (width 0.3) (layer "F.Cu") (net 7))
 (segment (start 42.75 5.5) (end 44.5 5.5) (width 0.3) (layer "F.Cu") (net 7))
 (segment (start 6.25 12) (end 6 12) (width 0.3) (layer "F.Cu") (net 7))
 (segment (start 5.5 9.5) (end 5.75 9.5) (width 0.3) (layer "F.Cu") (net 7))
 (segment (start 41.25 12.75) (end 6.25 12.75) (width 0.3) (layer "F.Cu") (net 7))
 (segment (start 5.75 9.5) (end 5.75 9.25) (width 0.3) (layer "F.Cu") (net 7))
 (segment (start 7 8) (end 7 8.08) (width 0.3) (layer "F.Cu") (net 7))
 (via (at 41.25 12.75) (size 0.8) (drill 0.4) (layers "F.Cu" "B.Cu") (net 7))
 (segment (start 41.25 6) (end 41.25 12.75) (width 0.3) (layer "B.Cu") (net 7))
 (segment (start 41.27 6) (end 41.25 6) (width 0.3) (layer "B.Cu") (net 7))
 (segment (start 9.5 10.25) (end 9.5 10.5) (width 0.3) (layer "F.Cu") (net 8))
 (segment (start 71.27 6) (end 71.25 6) (width 0.3) (layer "F.Cu") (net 8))
 (segment (start 75 4.75) (end 75 4.84) (width 0.3) (layer "F.Cu") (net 8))
 (segment (start 50 10.25) (end 9.5 10.25) (width 0.3) (layer "F.Cu") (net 8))
 (segment (start 74.5 5.25) (end 75 5.25) (width 0.3) (layer "F.Cu") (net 8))
 (segment (start 72.75 6) (end 72.75 5.5) (width 0.3) (layer "F.Cu") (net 8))
 (segment (start 74.5 5.5) (end 74.5 5.25) (width 0.3) (layer "F.Cu") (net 8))
 (segment (start 72.75 5.5) (end 74.5 5.5) (width 0.3) (layer "F.Cu") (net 8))
 (segment (start 9.5 10.5) (end 9.54 10.62) (width 0.3) (layer "F.Cu") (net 8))
 (segment (start 75 5.25) (end 75 4.75) (width 0.3) (layer "F.Cu") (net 8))
 (segment (start 71.25 6) (end 72.75 6) (width 0.3) (layer "F.Cu") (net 8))
 (via (at 50 10.25) (size 0.8) (drill 0.4) (layers "F.Cu" "B.Cu") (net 8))
 (segment (start 71.27 6) (end 71.25 6) (width 0.3) (layer "B.Cu") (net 8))
 (segment (start 59.25 10.25) (end 50 10.25) (width 0.3) (layer "B.Cu") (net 8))
 (segment (start 71.25 7.5) (end 70.75 7.5) (width 0.3) (layer "B.Cu") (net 8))
 (segment (start 59.25 8.5) (end 59.25 10.25) (width 0.3) (layer "B.Cu") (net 8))
 (segment (start 70.75 8.5) (end 59.25 8.5) (width 0.3) (layer "B.Cu") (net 8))
 (segment (start 70.75 7.5) (end 70.75 8.5) (width 0.3) (layer "B.Cu") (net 8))
 (segment (start 71.25 6) (end 71.25 7.5) (width 0.3) (layer "B.Cu") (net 8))
 (segment (start 19.5 4.25) (end 19.5 4) (width 0.3) (layer "F.Cu") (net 2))
 (segment (start 5.5 4.5) (end 5.75 4.5) (width 0.3) (layer "F.Cu") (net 2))
 (segment (start 6.25 1) (end 6.25 1.25) (width 0.3) (layer "F.Cu") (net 2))
 (segment (start 11.25 3.25) (end 11 3.25) (width 0.3) (layer "F.Cu") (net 2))
 (segment (start 5.25 3.75) (end 5.25 4.25) (width 0.3) (layer "F.Cu") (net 2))
 (segment (start 11.5 3.75) (end 11.5 3.5) (width 0.3) (layer "F.Cu") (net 2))
 (segment (start 7.75 1.25) (end 7.75 1) (width 0.3) (layer "F.Cu") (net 2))
 (segment (start 20.75 6) (end 20.75 4.5) (width 0.3) (layer "F.Cu") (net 2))
 (segment (start 5 3.75) (end 5.25 3.75) (width 0.3) (layer "F.Cu") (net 2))
 (segment (start 21.25 6) (end 20.75 6) (width 0.3) (layer "F.Cu") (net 2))
 (segment (start 7 5.5) (end 7 5.54) (width 0.3) (layer "F.Cu") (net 2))
 (segment (start 23.5 4.75) (end 23.5 5.25) (width 0.3) (layer "F.Cu") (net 2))
 (segment (start 25 4.75) (end 23.5 4.75) (width 0.3) (layer "F.Cu") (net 2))
 (segment (start 20 4.5) (end 20 4.25) (width 0.3) (layer "F.Cu") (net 2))
 (segment (start 5.75 4.5) (end 5.75 4.75) (width 0.3) (layer "F.Cu") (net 2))
 (segment (start 21.25 6) (end 21.27 6) (width 0.3) (layer "F.Cu") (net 2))
 (segment (start 5.5 1.5) (end 5.5 1.75) (width 0.3) (layer "F.Cu") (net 2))
 (segment (start 5.75 1.5) (end 5.5 1.5) (width 0.3) (layer "F.Cu") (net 2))
 (segment (start 20.75 4.5) (end 20 4.5) (width 0.3) (layer "F.Cu") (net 2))
 (segment (start 5.25 2.25) (end 5 2.25) (width 0.3) (layer "F.Cu") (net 2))
 (segment (start 10.5 1.5) (end 8.25 1.5) (width 0.3) (layer "F.Cu") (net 2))
 (segment (start 8.25 1.25) (end 7.75 1.25) (width 0.3) (layer "F.Cu") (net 2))
 (segment (start 10.75 1.75) (end 10.5 1.75) (width 0.3) (layer "F.Cu") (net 2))
 (segment (start 11.5 3.5) (end 11.25 3.5) (width 0.3) (layer "F.Cu") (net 2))
 (segment (start 11 2) (end 10.75 2) (width 0.3) (layer "F.Cu") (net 2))
 (segment (start 21.27 6) (end 21.25 6) (width 0.3) (layer "F.Cu") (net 2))
 (segment (start 5.25 1.75) (end 5.25 2.25) (width 0.3) (layer "F.Cu") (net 2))
 (segment (start 6.25 4.75) (end 6.25 5) (width 0.3) (layer "F.Cu") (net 2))
 (segment (start 10.75 2) (end 10.75 1.75) (width 0.3) (layer "F.Cu") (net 2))
 (segment (start 11.25 3.5) (end 11.25 3.25) (width 0.3) (layer "F.Cu") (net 2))
 (segment (start 19.5 4) (end 11.75 4) (width 0.3) (layer "F.Cu") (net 2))
 (segment (start 5 2.25) (end 5 3.75) (width 0.3) (layer "F.Cu") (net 2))
 (segment (start 23.5 5.25) (end 21.75 5.25) (width 0.3) (layer "F.Cu") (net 2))
 (segment (start 5.5 4.25) (end 5.5 4.5) (width 0.3) (layer "F.Cu") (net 2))
 (segment (start 11 3.25) (end 11 2) (width 0.3) (layer "F.Cu") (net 2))
 (segment (start 7.75 1) (end 6.25 1) (width 0.3) (layer "F.Cu") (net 2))
 (segment (start 7 5) (end 7 5.5) (width 0.3) (layer "F.Cu") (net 2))
 (segment (start 8.25 1.5) (end 8.25 1.25) (width 0.3) (layer "F.Cu") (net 2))
 (segment (start 11.75 3.75) (end 11.5 3.75) (width 0.3) (layer "F.Cu") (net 2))
 (segment (start 25 4.84) (end 25 4.75) (width 0.3) (layer "F.Cu") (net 2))
 (segment (start 21.75 5.25) (end 21.75 5.5) (width 0.3) (layer "F.Cu") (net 2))
 (segment (start 5.25 4.25) (end 5.5 4.25) (width 0.3) (layer "F.Cu") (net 2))
 (segment (start 5.75 4.75) (end 6.25 4.75) (width 0.3) (layer "F.Cu") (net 2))
 (segment (start 21.25 5.5) (end 21.25 6) (width 0.3) (layer "F.Cu") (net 2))
 (segment (start 11.75 4) (end 11.75 3.75) (width 0.3) (layer "F.Cu") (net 2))
 (segment (start 20 4.25) (end 19.5 4.25) (width 0.3) (layer "F.Cu") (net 2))
 (segment (start 6.25 5) (end 7 5) (width 0.3) (layer "F.Cu") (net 2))
 (segment (start 10.5 1.75) (end 10.5 1.5) (width 0.3) (layer "F.Cu") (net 2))
 (segment (start 21.75 5.5) (end 21.25 5.5) (width 0.3) (layer "F.Cu") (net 2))
 (segment (start 6.25 1.25) (end 5.75 1.25) (width 0.3) (layer "F.Cu") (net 2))
 (segment (start 5.5 1.75) (end 5.25 1.75) (width 0.3) (layer "F.Cu") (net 2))
 (segment (start 5.75 1.25) (end 5.75 1.5) (width 0.3) (layer "F.Cu") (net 2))
 (segment (start 35 4.84) (end 35 4.75) (width 0.3) (layer "F.Cu") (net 6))
 (segment (start 35 4.75) (end 33.5 4.75) (width 0.3) (layer "F.Cu") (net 6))
 (segment (start 33.5 4.75) (end 33.5 5.25) (width 0.3) (layer "F.Cu") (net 6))
 (segment (start 31.75 5.25) (end 31.75 5.5) (width 0.3) (layer "F.Cu") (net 6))
 (segment (start 31.25 5.5) (end 31.25 6) (width 0.3) (layer "F.Cu") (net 6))
 (segment (start 33.5 5.25) (end 31.75 5.25) (width 0.3) (layer "F.Cu") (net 6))
 (segment (start 31.25 6) (end 31.27 6) (width 0.3) (layer "F.Cu") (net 6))
 (segment (start 31.75 5.5) (end 31.25 5.5) (width 0.3) (layer "F.Cu") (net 6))
 (segment (start 29.5 7.75) (end 29.5 8) (width 0.3) (layer "B.Cu") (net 6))
 (segment (start 16.75 6.75) (end 16.75 5.5) (width 0.3) (layer "B.Cu") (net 6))
 (segment (start 9.5 5.5) (end 9.54 5.54) (width 0.3) (layer "B.Cu") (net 6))
 (segment (start 29.5 8) (end 18 8) (width 0.3) (layer "B.Cu") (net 6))
 (segment (start 31.27 6) (end 31.25 6) (width 0.3) (layer "B.Cu") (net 6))
 (segment (start 17.25 7.5) (end 17.25 7.25) (width 0.3) (layer "B.Cu") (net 6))
 (segment (start 18 7.75) (end 17.5 7.75) (width 0.3) (layer "B.Cu") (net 6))
 (segment (start 30.25 7.25) (end 30.25 7.5) (width 0.3) (layer "B.Cu") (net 6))
 (segment (start 30.25 7.5) (end 30 7.5) (width 0.3) (layer "B.Cu") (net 6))
 (segment (start 16.75 5.5) (end 9.5 5.5) (width 0.3) (layer "B.Cu") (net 6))
 (segment (start 30.75 6.75) (end 30.5 6.75) (width 0.3) (layer "B.Cu") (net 6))
 (segment (start 30.75 6) (end 30.75 6.75) (width 0.3) (layer "B.Cu") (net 6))
 (segment (start 17.25 7.25) (end 17 7.25) (width 0.3) (layer "B.Cu") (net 6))
 (segment (start 17 6.75) (end 16.75 6.75) (width 0.3) (layer "B.Cu") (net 6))
 (segment (start 30.5 7.25) (end 30.25 7.25) (width 0.3) (layer "B.Cu") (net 6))
 (segment (start 30 7.5) (end 30 7.75) (width 0.3) (layer "B.Cu") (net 6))
 (segment (start 30.5 6.75) (end 30.5 7.25) (width 0.3) (layer "B.Cu") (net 6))
 (segment (start 17.5 7.75) (end 17.5 7.5) (width 0.3) (layer "B.Cu") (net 6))
 (segment (start 30 7.75) (end 29.5 7.75) (width 0.3) (layer "B.Cu") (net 6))
 (segment (start 31.25 6) (end 30.75 6) (width 0.3) (layer "B.Cu") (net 6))
 (segment (start 17 7.25) (end 17 6.75) (width 0.3) (layer "B.Cu") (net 6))
 (segment (start 17.5 7.5) (end 17.25 7.5) (width 0.3) (layer "B.Cu") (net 6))
 (segment (start 18 8) (end 18 7.75) (width 0.3) (layer "B.Cu") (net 6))
 (segment (start 50 7.5) (end 50 7.75) (width 0.3) (layer "F.Cu") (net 5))
 (segment (start 43 8.25) (end 42.5 8.25) (width 0.3) (layer "F.Cu") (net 5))
 (segment (start 55 5.25) (end 55 4.75) (width 0.3) (layer "F.Cu") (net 5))
 (segment (start 50.75 6) (end 50.75 6.75) (width 0.3) (layer "F.Cu") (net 5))
 (segment (start 51.25 6) (end 50.75 6) (width 0.3) (layer "F.Cu") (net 5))
 (segment (start 50 7.75) (end 49.5 7.75) (width 0.3) (layer "F.Cu") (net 5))
 (segment (start 50.25 7.5) (end 50 7.5) (width 0.3) (layer "F.Cu") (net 5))
 (segment (start 50.75 6.75) (end 50.5 6.75) (width 0.3) (layer "F.Cu") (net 5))
 (segment (start 42.5 8.25) (end 42.5 8.5) (width 0.3) (layer "F.Cu") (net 5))
 (segment (start 50.5 6.75) (end 50.5 7.25) (width 0.3) (layer "F.Cu") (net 5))
 (segment (start 52.75 6) (end 52.75 5.5) (width 0.3) (layer "F.Cu") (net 5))
 (segment (start 9.5 8.5) (end 9.5 8) (width 0.3) (layer "F.Cu") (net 5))
 (segment (start 55 4.75) (end 55 4.84) (width 0.3) (layer "F.Cu") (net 5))
 (segment (start 52.75 5.5) (end 54.5 5.5) (width 0.3) (layer "F.Cu") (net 5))
 (segment (start 51.25 6) (end 52.75 6) (width 0.3) (layer "F.Cu") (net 5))
 (segment (start 43 8) (end 43 8.25) (width 0.3) (layer "F.Cu") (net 5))
 (segment (start 9.5 8) (end 9.54 8.08) (width 0.3) (layer "F.Cu") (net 5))
 (segment (start 51.27 6) (end 51.25 6) (width 0.3) (layer "F.Cu") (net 5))
 (segment (start 54.5 5.25) (end 55 5.25) (width 0.3) (layer "F.Cu") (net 5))
 (segment (start 50.25 7.25) (end 50.25 7.5) (width 0.3) (layer "F.Cu") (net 5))
 (segment (start 42.5 8.5) (end 9.5 8.5) (width 0.3) (layer "F.Cu") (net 5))
 (segment (start 54.5 5.5) (end 54.5 5.25) (width 0.3) (layer "F.Cu") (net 5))
 (segment (start 50.5 7.25) (end 50.25 7.25) (width 0.3) (layer "F.Cu") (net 5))
 (segment (start 49.5 8) (end 43 8) (width 0.3) (layer "F.Cu") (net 5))
 (segment (start 49.5 7.75) (end 49.5 8) (width 0.3) (layer "F.Cu") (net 5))
 (segment (start 51.27 6) (end 51.25 6) (width 0.3) (layer "F.Cu") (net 5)))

